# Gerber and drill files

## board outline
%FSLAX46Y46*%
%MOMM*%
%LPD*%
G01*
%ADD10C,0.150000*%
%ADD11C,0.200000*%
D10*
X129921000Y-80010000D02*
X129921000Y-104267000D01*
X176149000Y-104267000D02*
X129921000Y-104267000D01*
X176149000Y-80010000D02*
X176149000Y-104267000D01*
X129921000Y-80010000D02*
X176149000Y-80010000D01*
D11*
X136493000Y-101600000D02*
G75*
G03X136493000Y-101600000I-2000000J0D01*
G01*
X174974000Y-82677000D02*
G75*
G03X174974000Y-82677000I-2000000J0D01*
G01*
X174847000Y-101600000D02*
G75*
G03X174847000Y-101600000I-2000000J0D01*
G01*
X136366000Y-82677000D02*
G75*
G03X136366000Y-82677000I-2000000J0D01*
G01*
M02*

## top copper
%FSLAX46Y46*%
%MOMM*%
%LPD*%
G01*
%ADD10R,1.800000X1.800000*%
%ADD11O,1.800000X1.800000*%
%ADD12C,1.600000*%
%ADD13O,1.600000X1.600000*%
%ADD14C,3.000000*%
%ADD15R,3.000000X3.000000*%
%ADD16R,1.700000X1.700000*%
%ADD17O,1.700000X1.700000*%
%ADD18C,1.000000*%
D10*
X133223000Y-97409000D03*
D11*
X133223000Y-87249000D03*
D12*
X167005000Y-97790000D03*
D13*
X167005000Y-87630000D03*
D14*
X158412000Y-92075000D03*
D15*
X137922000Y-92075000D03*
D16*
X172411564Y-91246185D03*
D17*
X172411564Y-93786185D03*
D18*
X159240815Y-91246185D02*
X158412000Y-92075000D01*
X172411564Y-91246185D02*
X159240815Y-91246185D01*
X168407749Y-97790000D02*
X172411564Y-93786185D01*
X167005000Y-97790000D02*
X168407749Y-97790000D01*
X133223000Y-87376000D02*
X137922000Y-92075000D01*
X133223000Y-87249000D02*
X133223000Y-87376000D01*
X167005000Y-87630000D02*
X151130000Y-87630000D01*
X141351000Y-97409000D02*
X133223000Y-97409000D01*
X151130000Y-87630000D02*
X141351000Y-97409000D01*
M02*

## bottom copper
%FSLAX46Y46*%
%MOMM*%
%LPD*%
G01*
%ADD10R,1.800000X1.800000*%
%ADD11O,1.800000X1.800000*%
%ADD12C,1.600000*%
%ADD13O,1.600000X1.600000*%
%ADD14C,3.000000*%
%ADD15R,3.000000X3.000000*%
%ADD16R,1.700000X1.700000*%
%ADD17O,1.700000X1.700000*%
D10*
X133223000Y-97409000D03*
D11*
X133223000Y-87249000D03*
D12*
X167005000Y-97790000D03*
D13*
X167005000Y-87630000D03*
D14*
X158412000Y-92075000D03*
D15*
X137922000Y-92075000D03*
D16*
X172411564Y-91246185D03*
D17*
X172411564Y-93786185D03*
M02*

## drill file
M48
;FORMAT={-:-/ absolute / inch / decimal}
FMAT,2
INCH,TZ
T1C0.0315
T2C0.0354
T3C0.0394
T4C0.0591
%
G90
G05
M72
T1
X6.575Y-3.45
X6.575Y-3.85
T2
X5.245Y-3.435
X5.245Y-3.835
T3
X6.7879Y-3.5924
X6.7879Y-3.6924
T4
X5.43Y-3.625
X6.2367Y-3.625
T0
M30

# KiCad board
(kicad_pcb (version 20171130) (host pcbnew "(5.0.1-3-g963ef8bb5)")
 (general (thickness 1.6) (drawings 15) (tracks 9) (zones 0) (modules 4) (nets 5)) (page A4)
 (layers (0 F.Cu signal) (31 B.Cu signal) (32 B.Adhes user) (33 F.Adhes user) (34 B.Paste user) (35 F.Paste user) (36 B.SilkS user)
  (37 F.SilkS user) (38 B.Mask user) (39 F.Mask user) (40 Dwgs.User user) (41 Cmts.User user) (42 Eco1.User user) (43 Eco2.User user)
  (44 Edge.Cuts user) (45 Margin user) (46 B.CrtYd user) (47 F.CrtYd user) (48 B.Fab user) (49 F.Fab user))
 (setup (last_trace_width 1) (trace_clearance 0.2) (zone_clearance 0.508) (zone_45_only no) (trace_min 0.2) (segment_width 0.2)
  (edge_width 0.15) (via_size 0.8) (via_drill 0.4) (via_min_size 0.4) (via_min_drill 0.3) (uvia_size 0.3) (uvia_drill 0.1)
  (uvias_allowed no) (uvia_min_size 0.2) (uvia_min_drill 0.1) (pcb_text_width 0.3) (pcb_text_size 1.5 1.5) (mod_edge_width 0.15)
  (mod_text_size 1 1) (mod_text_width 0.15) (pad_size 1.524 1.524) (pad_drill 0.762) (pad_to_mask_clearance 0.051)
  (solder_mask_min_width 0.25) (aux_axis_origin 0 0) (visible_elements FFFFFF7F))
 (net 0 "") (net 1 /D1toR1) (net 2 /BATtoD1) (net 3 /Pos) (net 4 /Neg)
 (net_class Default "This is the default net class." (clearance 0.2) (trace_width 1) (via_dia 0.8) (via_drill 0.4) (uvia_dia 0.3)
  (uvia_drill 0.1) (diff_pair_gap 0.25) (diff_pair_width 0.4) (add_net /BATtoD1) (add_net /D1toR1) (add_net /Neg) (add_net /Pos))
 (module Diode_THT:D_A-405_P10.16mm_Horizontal (layer F.Cu) (at 133.223 97.409 90)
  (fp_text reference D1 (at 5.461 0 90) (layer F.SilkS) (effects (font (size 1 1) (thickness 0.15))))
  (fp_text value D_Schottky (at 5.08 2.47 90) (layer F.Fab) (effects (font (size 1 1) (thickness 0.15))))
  (pad 1 thru_hole rect (at 0 0 90) (size 1.8 1.8) (drill 0.9) (layers *.Cu *.Mask) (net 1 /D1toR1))
  (pad 2 thru_hole oval (at 10.16 0 90) (size 1.8 1.8) (drill 0.9) (layers *.Cu *.Mask) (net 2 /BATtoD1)))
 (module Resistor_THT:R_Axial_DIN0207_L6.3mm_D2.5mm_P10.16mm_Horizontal (layer F.Cu) (at 167.005 97.79 90)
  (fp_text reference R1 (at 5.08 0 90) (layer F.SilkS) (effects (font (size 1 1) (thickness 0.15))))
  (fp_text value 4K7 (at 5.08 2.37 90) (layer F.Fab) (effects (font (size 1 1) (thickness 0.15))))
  (pad 1 thru_hole circle (at 0 0 90) (size 1.6 1.6) (drill 0.8) (layers *.Cu *.Mask) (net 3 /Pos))
  (pad 2 thru_hole oval (at 10.16 0 90) (size 1.6 1.6) (drill 0.8) (layers *.Cu *.Mask) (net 1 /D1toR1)))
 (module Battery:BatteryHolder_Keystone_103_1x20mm (layer F.Cu) (at 137.922 92.075)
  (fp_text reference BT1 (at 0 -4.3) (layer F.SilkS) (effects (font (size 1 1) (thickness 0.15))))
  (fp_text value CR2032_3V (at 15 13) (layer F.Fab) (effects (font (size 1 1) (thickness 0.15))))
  (pad 2 thru_hole circle (at 20.49 0) (size 3 3) (drill 1.5) (layers *.Cu *.Mask) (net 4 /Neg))
  (pad 1 thru_hole rect (at 0 0) (size 3 3) (drill 1.5) (layers *.Cu *.Mask) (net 2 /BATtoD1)))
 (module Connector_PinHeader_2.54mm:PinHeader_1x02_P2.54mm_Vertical (layer F.Cu) (at 172.411564 91.246185)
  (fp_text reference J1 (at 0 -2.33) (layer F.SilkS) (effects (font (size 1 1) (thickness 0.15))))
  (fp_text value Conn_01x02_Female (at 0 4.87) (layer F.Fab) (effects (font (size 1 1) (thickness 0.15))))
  (pad 1 thru_hole rect (at 0 0) (size 1.7 1.7) (drill 1) (layers *.Cu *.Mask) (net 4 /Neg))
  (pad 2 thru_hole oval (at 0 2.54) (size 1.7 1.7) (drill 1) (layers *.Cu *.Mask) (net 3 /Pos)))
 (gr_line (start 129.921 80.01) (end 129.921 104.267) (layer Edge.Cuts) (width 0.15))
 (gr_line (start 176.149 104.267) (end 129.921 104.267) (layer Edge.Cuts) (width 0.15))
 (gr_line (start 176.149 80.01) (end 176.149 104.267) (layer Edge.Cuts) (width 0.15))
 (gr_line (start 129.921 80.01) (end 176.149 80.01) (layer Edge.Cuts) (width 0.15))
 (gr_circle (center 134.493 101.6) (end 136.493 101.6) (layer Edge.Cuts) (width 0.2))
 (gr_circle (center 172.974 82.677) (end 174.974 82.677) (layer Edge.Cuts) (width 0.2))
 (gr_circle (center 172.847 101.6) (end 174.847 101.6) (layer Edge.Cuts) (width 0.2))
 (gr_circle (center 134.366 82.677) (end 136.366 82.677) (layer Edge.Cuts) (width 0.2))
 (segment (start 159.240815 91.246185) (end 158.412 92.075) (width 1) (layer F.Cu) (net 4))
 (segment (start 172.411564 91.246185) (end 159.240815 91.246185) (width 1) (layer F.Cu) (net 4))
 (segment (start 168.407749 97.79) (end 172.411564 93.786185) (width 1) (layer F.Cu) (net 3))
 (segment (start 167.005 97.79) (end 168.407749 97.79) (width 1) (layer F.Cu) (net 3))
 (segment (start 133.223 87.376) (end 137.922 92.075) (width 1) (layer F.Cu) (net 2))
 (segment (start 133.223 87.249) (end 133.223 87.376) (width 1) (layer F.Cu) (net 2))
 (segment (start 167.005 87.63) (end 151.13 87.63) (width 1) (layer F.Cu) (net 1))
 (segment (start 141.351 97.409) (end 133.223 97.409) (width 1) (layer F.Cu) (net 1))
 (segment (start 151.13 87.63) (end 141.351 97.409) (width 1) (layer F.Cu) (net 1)))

